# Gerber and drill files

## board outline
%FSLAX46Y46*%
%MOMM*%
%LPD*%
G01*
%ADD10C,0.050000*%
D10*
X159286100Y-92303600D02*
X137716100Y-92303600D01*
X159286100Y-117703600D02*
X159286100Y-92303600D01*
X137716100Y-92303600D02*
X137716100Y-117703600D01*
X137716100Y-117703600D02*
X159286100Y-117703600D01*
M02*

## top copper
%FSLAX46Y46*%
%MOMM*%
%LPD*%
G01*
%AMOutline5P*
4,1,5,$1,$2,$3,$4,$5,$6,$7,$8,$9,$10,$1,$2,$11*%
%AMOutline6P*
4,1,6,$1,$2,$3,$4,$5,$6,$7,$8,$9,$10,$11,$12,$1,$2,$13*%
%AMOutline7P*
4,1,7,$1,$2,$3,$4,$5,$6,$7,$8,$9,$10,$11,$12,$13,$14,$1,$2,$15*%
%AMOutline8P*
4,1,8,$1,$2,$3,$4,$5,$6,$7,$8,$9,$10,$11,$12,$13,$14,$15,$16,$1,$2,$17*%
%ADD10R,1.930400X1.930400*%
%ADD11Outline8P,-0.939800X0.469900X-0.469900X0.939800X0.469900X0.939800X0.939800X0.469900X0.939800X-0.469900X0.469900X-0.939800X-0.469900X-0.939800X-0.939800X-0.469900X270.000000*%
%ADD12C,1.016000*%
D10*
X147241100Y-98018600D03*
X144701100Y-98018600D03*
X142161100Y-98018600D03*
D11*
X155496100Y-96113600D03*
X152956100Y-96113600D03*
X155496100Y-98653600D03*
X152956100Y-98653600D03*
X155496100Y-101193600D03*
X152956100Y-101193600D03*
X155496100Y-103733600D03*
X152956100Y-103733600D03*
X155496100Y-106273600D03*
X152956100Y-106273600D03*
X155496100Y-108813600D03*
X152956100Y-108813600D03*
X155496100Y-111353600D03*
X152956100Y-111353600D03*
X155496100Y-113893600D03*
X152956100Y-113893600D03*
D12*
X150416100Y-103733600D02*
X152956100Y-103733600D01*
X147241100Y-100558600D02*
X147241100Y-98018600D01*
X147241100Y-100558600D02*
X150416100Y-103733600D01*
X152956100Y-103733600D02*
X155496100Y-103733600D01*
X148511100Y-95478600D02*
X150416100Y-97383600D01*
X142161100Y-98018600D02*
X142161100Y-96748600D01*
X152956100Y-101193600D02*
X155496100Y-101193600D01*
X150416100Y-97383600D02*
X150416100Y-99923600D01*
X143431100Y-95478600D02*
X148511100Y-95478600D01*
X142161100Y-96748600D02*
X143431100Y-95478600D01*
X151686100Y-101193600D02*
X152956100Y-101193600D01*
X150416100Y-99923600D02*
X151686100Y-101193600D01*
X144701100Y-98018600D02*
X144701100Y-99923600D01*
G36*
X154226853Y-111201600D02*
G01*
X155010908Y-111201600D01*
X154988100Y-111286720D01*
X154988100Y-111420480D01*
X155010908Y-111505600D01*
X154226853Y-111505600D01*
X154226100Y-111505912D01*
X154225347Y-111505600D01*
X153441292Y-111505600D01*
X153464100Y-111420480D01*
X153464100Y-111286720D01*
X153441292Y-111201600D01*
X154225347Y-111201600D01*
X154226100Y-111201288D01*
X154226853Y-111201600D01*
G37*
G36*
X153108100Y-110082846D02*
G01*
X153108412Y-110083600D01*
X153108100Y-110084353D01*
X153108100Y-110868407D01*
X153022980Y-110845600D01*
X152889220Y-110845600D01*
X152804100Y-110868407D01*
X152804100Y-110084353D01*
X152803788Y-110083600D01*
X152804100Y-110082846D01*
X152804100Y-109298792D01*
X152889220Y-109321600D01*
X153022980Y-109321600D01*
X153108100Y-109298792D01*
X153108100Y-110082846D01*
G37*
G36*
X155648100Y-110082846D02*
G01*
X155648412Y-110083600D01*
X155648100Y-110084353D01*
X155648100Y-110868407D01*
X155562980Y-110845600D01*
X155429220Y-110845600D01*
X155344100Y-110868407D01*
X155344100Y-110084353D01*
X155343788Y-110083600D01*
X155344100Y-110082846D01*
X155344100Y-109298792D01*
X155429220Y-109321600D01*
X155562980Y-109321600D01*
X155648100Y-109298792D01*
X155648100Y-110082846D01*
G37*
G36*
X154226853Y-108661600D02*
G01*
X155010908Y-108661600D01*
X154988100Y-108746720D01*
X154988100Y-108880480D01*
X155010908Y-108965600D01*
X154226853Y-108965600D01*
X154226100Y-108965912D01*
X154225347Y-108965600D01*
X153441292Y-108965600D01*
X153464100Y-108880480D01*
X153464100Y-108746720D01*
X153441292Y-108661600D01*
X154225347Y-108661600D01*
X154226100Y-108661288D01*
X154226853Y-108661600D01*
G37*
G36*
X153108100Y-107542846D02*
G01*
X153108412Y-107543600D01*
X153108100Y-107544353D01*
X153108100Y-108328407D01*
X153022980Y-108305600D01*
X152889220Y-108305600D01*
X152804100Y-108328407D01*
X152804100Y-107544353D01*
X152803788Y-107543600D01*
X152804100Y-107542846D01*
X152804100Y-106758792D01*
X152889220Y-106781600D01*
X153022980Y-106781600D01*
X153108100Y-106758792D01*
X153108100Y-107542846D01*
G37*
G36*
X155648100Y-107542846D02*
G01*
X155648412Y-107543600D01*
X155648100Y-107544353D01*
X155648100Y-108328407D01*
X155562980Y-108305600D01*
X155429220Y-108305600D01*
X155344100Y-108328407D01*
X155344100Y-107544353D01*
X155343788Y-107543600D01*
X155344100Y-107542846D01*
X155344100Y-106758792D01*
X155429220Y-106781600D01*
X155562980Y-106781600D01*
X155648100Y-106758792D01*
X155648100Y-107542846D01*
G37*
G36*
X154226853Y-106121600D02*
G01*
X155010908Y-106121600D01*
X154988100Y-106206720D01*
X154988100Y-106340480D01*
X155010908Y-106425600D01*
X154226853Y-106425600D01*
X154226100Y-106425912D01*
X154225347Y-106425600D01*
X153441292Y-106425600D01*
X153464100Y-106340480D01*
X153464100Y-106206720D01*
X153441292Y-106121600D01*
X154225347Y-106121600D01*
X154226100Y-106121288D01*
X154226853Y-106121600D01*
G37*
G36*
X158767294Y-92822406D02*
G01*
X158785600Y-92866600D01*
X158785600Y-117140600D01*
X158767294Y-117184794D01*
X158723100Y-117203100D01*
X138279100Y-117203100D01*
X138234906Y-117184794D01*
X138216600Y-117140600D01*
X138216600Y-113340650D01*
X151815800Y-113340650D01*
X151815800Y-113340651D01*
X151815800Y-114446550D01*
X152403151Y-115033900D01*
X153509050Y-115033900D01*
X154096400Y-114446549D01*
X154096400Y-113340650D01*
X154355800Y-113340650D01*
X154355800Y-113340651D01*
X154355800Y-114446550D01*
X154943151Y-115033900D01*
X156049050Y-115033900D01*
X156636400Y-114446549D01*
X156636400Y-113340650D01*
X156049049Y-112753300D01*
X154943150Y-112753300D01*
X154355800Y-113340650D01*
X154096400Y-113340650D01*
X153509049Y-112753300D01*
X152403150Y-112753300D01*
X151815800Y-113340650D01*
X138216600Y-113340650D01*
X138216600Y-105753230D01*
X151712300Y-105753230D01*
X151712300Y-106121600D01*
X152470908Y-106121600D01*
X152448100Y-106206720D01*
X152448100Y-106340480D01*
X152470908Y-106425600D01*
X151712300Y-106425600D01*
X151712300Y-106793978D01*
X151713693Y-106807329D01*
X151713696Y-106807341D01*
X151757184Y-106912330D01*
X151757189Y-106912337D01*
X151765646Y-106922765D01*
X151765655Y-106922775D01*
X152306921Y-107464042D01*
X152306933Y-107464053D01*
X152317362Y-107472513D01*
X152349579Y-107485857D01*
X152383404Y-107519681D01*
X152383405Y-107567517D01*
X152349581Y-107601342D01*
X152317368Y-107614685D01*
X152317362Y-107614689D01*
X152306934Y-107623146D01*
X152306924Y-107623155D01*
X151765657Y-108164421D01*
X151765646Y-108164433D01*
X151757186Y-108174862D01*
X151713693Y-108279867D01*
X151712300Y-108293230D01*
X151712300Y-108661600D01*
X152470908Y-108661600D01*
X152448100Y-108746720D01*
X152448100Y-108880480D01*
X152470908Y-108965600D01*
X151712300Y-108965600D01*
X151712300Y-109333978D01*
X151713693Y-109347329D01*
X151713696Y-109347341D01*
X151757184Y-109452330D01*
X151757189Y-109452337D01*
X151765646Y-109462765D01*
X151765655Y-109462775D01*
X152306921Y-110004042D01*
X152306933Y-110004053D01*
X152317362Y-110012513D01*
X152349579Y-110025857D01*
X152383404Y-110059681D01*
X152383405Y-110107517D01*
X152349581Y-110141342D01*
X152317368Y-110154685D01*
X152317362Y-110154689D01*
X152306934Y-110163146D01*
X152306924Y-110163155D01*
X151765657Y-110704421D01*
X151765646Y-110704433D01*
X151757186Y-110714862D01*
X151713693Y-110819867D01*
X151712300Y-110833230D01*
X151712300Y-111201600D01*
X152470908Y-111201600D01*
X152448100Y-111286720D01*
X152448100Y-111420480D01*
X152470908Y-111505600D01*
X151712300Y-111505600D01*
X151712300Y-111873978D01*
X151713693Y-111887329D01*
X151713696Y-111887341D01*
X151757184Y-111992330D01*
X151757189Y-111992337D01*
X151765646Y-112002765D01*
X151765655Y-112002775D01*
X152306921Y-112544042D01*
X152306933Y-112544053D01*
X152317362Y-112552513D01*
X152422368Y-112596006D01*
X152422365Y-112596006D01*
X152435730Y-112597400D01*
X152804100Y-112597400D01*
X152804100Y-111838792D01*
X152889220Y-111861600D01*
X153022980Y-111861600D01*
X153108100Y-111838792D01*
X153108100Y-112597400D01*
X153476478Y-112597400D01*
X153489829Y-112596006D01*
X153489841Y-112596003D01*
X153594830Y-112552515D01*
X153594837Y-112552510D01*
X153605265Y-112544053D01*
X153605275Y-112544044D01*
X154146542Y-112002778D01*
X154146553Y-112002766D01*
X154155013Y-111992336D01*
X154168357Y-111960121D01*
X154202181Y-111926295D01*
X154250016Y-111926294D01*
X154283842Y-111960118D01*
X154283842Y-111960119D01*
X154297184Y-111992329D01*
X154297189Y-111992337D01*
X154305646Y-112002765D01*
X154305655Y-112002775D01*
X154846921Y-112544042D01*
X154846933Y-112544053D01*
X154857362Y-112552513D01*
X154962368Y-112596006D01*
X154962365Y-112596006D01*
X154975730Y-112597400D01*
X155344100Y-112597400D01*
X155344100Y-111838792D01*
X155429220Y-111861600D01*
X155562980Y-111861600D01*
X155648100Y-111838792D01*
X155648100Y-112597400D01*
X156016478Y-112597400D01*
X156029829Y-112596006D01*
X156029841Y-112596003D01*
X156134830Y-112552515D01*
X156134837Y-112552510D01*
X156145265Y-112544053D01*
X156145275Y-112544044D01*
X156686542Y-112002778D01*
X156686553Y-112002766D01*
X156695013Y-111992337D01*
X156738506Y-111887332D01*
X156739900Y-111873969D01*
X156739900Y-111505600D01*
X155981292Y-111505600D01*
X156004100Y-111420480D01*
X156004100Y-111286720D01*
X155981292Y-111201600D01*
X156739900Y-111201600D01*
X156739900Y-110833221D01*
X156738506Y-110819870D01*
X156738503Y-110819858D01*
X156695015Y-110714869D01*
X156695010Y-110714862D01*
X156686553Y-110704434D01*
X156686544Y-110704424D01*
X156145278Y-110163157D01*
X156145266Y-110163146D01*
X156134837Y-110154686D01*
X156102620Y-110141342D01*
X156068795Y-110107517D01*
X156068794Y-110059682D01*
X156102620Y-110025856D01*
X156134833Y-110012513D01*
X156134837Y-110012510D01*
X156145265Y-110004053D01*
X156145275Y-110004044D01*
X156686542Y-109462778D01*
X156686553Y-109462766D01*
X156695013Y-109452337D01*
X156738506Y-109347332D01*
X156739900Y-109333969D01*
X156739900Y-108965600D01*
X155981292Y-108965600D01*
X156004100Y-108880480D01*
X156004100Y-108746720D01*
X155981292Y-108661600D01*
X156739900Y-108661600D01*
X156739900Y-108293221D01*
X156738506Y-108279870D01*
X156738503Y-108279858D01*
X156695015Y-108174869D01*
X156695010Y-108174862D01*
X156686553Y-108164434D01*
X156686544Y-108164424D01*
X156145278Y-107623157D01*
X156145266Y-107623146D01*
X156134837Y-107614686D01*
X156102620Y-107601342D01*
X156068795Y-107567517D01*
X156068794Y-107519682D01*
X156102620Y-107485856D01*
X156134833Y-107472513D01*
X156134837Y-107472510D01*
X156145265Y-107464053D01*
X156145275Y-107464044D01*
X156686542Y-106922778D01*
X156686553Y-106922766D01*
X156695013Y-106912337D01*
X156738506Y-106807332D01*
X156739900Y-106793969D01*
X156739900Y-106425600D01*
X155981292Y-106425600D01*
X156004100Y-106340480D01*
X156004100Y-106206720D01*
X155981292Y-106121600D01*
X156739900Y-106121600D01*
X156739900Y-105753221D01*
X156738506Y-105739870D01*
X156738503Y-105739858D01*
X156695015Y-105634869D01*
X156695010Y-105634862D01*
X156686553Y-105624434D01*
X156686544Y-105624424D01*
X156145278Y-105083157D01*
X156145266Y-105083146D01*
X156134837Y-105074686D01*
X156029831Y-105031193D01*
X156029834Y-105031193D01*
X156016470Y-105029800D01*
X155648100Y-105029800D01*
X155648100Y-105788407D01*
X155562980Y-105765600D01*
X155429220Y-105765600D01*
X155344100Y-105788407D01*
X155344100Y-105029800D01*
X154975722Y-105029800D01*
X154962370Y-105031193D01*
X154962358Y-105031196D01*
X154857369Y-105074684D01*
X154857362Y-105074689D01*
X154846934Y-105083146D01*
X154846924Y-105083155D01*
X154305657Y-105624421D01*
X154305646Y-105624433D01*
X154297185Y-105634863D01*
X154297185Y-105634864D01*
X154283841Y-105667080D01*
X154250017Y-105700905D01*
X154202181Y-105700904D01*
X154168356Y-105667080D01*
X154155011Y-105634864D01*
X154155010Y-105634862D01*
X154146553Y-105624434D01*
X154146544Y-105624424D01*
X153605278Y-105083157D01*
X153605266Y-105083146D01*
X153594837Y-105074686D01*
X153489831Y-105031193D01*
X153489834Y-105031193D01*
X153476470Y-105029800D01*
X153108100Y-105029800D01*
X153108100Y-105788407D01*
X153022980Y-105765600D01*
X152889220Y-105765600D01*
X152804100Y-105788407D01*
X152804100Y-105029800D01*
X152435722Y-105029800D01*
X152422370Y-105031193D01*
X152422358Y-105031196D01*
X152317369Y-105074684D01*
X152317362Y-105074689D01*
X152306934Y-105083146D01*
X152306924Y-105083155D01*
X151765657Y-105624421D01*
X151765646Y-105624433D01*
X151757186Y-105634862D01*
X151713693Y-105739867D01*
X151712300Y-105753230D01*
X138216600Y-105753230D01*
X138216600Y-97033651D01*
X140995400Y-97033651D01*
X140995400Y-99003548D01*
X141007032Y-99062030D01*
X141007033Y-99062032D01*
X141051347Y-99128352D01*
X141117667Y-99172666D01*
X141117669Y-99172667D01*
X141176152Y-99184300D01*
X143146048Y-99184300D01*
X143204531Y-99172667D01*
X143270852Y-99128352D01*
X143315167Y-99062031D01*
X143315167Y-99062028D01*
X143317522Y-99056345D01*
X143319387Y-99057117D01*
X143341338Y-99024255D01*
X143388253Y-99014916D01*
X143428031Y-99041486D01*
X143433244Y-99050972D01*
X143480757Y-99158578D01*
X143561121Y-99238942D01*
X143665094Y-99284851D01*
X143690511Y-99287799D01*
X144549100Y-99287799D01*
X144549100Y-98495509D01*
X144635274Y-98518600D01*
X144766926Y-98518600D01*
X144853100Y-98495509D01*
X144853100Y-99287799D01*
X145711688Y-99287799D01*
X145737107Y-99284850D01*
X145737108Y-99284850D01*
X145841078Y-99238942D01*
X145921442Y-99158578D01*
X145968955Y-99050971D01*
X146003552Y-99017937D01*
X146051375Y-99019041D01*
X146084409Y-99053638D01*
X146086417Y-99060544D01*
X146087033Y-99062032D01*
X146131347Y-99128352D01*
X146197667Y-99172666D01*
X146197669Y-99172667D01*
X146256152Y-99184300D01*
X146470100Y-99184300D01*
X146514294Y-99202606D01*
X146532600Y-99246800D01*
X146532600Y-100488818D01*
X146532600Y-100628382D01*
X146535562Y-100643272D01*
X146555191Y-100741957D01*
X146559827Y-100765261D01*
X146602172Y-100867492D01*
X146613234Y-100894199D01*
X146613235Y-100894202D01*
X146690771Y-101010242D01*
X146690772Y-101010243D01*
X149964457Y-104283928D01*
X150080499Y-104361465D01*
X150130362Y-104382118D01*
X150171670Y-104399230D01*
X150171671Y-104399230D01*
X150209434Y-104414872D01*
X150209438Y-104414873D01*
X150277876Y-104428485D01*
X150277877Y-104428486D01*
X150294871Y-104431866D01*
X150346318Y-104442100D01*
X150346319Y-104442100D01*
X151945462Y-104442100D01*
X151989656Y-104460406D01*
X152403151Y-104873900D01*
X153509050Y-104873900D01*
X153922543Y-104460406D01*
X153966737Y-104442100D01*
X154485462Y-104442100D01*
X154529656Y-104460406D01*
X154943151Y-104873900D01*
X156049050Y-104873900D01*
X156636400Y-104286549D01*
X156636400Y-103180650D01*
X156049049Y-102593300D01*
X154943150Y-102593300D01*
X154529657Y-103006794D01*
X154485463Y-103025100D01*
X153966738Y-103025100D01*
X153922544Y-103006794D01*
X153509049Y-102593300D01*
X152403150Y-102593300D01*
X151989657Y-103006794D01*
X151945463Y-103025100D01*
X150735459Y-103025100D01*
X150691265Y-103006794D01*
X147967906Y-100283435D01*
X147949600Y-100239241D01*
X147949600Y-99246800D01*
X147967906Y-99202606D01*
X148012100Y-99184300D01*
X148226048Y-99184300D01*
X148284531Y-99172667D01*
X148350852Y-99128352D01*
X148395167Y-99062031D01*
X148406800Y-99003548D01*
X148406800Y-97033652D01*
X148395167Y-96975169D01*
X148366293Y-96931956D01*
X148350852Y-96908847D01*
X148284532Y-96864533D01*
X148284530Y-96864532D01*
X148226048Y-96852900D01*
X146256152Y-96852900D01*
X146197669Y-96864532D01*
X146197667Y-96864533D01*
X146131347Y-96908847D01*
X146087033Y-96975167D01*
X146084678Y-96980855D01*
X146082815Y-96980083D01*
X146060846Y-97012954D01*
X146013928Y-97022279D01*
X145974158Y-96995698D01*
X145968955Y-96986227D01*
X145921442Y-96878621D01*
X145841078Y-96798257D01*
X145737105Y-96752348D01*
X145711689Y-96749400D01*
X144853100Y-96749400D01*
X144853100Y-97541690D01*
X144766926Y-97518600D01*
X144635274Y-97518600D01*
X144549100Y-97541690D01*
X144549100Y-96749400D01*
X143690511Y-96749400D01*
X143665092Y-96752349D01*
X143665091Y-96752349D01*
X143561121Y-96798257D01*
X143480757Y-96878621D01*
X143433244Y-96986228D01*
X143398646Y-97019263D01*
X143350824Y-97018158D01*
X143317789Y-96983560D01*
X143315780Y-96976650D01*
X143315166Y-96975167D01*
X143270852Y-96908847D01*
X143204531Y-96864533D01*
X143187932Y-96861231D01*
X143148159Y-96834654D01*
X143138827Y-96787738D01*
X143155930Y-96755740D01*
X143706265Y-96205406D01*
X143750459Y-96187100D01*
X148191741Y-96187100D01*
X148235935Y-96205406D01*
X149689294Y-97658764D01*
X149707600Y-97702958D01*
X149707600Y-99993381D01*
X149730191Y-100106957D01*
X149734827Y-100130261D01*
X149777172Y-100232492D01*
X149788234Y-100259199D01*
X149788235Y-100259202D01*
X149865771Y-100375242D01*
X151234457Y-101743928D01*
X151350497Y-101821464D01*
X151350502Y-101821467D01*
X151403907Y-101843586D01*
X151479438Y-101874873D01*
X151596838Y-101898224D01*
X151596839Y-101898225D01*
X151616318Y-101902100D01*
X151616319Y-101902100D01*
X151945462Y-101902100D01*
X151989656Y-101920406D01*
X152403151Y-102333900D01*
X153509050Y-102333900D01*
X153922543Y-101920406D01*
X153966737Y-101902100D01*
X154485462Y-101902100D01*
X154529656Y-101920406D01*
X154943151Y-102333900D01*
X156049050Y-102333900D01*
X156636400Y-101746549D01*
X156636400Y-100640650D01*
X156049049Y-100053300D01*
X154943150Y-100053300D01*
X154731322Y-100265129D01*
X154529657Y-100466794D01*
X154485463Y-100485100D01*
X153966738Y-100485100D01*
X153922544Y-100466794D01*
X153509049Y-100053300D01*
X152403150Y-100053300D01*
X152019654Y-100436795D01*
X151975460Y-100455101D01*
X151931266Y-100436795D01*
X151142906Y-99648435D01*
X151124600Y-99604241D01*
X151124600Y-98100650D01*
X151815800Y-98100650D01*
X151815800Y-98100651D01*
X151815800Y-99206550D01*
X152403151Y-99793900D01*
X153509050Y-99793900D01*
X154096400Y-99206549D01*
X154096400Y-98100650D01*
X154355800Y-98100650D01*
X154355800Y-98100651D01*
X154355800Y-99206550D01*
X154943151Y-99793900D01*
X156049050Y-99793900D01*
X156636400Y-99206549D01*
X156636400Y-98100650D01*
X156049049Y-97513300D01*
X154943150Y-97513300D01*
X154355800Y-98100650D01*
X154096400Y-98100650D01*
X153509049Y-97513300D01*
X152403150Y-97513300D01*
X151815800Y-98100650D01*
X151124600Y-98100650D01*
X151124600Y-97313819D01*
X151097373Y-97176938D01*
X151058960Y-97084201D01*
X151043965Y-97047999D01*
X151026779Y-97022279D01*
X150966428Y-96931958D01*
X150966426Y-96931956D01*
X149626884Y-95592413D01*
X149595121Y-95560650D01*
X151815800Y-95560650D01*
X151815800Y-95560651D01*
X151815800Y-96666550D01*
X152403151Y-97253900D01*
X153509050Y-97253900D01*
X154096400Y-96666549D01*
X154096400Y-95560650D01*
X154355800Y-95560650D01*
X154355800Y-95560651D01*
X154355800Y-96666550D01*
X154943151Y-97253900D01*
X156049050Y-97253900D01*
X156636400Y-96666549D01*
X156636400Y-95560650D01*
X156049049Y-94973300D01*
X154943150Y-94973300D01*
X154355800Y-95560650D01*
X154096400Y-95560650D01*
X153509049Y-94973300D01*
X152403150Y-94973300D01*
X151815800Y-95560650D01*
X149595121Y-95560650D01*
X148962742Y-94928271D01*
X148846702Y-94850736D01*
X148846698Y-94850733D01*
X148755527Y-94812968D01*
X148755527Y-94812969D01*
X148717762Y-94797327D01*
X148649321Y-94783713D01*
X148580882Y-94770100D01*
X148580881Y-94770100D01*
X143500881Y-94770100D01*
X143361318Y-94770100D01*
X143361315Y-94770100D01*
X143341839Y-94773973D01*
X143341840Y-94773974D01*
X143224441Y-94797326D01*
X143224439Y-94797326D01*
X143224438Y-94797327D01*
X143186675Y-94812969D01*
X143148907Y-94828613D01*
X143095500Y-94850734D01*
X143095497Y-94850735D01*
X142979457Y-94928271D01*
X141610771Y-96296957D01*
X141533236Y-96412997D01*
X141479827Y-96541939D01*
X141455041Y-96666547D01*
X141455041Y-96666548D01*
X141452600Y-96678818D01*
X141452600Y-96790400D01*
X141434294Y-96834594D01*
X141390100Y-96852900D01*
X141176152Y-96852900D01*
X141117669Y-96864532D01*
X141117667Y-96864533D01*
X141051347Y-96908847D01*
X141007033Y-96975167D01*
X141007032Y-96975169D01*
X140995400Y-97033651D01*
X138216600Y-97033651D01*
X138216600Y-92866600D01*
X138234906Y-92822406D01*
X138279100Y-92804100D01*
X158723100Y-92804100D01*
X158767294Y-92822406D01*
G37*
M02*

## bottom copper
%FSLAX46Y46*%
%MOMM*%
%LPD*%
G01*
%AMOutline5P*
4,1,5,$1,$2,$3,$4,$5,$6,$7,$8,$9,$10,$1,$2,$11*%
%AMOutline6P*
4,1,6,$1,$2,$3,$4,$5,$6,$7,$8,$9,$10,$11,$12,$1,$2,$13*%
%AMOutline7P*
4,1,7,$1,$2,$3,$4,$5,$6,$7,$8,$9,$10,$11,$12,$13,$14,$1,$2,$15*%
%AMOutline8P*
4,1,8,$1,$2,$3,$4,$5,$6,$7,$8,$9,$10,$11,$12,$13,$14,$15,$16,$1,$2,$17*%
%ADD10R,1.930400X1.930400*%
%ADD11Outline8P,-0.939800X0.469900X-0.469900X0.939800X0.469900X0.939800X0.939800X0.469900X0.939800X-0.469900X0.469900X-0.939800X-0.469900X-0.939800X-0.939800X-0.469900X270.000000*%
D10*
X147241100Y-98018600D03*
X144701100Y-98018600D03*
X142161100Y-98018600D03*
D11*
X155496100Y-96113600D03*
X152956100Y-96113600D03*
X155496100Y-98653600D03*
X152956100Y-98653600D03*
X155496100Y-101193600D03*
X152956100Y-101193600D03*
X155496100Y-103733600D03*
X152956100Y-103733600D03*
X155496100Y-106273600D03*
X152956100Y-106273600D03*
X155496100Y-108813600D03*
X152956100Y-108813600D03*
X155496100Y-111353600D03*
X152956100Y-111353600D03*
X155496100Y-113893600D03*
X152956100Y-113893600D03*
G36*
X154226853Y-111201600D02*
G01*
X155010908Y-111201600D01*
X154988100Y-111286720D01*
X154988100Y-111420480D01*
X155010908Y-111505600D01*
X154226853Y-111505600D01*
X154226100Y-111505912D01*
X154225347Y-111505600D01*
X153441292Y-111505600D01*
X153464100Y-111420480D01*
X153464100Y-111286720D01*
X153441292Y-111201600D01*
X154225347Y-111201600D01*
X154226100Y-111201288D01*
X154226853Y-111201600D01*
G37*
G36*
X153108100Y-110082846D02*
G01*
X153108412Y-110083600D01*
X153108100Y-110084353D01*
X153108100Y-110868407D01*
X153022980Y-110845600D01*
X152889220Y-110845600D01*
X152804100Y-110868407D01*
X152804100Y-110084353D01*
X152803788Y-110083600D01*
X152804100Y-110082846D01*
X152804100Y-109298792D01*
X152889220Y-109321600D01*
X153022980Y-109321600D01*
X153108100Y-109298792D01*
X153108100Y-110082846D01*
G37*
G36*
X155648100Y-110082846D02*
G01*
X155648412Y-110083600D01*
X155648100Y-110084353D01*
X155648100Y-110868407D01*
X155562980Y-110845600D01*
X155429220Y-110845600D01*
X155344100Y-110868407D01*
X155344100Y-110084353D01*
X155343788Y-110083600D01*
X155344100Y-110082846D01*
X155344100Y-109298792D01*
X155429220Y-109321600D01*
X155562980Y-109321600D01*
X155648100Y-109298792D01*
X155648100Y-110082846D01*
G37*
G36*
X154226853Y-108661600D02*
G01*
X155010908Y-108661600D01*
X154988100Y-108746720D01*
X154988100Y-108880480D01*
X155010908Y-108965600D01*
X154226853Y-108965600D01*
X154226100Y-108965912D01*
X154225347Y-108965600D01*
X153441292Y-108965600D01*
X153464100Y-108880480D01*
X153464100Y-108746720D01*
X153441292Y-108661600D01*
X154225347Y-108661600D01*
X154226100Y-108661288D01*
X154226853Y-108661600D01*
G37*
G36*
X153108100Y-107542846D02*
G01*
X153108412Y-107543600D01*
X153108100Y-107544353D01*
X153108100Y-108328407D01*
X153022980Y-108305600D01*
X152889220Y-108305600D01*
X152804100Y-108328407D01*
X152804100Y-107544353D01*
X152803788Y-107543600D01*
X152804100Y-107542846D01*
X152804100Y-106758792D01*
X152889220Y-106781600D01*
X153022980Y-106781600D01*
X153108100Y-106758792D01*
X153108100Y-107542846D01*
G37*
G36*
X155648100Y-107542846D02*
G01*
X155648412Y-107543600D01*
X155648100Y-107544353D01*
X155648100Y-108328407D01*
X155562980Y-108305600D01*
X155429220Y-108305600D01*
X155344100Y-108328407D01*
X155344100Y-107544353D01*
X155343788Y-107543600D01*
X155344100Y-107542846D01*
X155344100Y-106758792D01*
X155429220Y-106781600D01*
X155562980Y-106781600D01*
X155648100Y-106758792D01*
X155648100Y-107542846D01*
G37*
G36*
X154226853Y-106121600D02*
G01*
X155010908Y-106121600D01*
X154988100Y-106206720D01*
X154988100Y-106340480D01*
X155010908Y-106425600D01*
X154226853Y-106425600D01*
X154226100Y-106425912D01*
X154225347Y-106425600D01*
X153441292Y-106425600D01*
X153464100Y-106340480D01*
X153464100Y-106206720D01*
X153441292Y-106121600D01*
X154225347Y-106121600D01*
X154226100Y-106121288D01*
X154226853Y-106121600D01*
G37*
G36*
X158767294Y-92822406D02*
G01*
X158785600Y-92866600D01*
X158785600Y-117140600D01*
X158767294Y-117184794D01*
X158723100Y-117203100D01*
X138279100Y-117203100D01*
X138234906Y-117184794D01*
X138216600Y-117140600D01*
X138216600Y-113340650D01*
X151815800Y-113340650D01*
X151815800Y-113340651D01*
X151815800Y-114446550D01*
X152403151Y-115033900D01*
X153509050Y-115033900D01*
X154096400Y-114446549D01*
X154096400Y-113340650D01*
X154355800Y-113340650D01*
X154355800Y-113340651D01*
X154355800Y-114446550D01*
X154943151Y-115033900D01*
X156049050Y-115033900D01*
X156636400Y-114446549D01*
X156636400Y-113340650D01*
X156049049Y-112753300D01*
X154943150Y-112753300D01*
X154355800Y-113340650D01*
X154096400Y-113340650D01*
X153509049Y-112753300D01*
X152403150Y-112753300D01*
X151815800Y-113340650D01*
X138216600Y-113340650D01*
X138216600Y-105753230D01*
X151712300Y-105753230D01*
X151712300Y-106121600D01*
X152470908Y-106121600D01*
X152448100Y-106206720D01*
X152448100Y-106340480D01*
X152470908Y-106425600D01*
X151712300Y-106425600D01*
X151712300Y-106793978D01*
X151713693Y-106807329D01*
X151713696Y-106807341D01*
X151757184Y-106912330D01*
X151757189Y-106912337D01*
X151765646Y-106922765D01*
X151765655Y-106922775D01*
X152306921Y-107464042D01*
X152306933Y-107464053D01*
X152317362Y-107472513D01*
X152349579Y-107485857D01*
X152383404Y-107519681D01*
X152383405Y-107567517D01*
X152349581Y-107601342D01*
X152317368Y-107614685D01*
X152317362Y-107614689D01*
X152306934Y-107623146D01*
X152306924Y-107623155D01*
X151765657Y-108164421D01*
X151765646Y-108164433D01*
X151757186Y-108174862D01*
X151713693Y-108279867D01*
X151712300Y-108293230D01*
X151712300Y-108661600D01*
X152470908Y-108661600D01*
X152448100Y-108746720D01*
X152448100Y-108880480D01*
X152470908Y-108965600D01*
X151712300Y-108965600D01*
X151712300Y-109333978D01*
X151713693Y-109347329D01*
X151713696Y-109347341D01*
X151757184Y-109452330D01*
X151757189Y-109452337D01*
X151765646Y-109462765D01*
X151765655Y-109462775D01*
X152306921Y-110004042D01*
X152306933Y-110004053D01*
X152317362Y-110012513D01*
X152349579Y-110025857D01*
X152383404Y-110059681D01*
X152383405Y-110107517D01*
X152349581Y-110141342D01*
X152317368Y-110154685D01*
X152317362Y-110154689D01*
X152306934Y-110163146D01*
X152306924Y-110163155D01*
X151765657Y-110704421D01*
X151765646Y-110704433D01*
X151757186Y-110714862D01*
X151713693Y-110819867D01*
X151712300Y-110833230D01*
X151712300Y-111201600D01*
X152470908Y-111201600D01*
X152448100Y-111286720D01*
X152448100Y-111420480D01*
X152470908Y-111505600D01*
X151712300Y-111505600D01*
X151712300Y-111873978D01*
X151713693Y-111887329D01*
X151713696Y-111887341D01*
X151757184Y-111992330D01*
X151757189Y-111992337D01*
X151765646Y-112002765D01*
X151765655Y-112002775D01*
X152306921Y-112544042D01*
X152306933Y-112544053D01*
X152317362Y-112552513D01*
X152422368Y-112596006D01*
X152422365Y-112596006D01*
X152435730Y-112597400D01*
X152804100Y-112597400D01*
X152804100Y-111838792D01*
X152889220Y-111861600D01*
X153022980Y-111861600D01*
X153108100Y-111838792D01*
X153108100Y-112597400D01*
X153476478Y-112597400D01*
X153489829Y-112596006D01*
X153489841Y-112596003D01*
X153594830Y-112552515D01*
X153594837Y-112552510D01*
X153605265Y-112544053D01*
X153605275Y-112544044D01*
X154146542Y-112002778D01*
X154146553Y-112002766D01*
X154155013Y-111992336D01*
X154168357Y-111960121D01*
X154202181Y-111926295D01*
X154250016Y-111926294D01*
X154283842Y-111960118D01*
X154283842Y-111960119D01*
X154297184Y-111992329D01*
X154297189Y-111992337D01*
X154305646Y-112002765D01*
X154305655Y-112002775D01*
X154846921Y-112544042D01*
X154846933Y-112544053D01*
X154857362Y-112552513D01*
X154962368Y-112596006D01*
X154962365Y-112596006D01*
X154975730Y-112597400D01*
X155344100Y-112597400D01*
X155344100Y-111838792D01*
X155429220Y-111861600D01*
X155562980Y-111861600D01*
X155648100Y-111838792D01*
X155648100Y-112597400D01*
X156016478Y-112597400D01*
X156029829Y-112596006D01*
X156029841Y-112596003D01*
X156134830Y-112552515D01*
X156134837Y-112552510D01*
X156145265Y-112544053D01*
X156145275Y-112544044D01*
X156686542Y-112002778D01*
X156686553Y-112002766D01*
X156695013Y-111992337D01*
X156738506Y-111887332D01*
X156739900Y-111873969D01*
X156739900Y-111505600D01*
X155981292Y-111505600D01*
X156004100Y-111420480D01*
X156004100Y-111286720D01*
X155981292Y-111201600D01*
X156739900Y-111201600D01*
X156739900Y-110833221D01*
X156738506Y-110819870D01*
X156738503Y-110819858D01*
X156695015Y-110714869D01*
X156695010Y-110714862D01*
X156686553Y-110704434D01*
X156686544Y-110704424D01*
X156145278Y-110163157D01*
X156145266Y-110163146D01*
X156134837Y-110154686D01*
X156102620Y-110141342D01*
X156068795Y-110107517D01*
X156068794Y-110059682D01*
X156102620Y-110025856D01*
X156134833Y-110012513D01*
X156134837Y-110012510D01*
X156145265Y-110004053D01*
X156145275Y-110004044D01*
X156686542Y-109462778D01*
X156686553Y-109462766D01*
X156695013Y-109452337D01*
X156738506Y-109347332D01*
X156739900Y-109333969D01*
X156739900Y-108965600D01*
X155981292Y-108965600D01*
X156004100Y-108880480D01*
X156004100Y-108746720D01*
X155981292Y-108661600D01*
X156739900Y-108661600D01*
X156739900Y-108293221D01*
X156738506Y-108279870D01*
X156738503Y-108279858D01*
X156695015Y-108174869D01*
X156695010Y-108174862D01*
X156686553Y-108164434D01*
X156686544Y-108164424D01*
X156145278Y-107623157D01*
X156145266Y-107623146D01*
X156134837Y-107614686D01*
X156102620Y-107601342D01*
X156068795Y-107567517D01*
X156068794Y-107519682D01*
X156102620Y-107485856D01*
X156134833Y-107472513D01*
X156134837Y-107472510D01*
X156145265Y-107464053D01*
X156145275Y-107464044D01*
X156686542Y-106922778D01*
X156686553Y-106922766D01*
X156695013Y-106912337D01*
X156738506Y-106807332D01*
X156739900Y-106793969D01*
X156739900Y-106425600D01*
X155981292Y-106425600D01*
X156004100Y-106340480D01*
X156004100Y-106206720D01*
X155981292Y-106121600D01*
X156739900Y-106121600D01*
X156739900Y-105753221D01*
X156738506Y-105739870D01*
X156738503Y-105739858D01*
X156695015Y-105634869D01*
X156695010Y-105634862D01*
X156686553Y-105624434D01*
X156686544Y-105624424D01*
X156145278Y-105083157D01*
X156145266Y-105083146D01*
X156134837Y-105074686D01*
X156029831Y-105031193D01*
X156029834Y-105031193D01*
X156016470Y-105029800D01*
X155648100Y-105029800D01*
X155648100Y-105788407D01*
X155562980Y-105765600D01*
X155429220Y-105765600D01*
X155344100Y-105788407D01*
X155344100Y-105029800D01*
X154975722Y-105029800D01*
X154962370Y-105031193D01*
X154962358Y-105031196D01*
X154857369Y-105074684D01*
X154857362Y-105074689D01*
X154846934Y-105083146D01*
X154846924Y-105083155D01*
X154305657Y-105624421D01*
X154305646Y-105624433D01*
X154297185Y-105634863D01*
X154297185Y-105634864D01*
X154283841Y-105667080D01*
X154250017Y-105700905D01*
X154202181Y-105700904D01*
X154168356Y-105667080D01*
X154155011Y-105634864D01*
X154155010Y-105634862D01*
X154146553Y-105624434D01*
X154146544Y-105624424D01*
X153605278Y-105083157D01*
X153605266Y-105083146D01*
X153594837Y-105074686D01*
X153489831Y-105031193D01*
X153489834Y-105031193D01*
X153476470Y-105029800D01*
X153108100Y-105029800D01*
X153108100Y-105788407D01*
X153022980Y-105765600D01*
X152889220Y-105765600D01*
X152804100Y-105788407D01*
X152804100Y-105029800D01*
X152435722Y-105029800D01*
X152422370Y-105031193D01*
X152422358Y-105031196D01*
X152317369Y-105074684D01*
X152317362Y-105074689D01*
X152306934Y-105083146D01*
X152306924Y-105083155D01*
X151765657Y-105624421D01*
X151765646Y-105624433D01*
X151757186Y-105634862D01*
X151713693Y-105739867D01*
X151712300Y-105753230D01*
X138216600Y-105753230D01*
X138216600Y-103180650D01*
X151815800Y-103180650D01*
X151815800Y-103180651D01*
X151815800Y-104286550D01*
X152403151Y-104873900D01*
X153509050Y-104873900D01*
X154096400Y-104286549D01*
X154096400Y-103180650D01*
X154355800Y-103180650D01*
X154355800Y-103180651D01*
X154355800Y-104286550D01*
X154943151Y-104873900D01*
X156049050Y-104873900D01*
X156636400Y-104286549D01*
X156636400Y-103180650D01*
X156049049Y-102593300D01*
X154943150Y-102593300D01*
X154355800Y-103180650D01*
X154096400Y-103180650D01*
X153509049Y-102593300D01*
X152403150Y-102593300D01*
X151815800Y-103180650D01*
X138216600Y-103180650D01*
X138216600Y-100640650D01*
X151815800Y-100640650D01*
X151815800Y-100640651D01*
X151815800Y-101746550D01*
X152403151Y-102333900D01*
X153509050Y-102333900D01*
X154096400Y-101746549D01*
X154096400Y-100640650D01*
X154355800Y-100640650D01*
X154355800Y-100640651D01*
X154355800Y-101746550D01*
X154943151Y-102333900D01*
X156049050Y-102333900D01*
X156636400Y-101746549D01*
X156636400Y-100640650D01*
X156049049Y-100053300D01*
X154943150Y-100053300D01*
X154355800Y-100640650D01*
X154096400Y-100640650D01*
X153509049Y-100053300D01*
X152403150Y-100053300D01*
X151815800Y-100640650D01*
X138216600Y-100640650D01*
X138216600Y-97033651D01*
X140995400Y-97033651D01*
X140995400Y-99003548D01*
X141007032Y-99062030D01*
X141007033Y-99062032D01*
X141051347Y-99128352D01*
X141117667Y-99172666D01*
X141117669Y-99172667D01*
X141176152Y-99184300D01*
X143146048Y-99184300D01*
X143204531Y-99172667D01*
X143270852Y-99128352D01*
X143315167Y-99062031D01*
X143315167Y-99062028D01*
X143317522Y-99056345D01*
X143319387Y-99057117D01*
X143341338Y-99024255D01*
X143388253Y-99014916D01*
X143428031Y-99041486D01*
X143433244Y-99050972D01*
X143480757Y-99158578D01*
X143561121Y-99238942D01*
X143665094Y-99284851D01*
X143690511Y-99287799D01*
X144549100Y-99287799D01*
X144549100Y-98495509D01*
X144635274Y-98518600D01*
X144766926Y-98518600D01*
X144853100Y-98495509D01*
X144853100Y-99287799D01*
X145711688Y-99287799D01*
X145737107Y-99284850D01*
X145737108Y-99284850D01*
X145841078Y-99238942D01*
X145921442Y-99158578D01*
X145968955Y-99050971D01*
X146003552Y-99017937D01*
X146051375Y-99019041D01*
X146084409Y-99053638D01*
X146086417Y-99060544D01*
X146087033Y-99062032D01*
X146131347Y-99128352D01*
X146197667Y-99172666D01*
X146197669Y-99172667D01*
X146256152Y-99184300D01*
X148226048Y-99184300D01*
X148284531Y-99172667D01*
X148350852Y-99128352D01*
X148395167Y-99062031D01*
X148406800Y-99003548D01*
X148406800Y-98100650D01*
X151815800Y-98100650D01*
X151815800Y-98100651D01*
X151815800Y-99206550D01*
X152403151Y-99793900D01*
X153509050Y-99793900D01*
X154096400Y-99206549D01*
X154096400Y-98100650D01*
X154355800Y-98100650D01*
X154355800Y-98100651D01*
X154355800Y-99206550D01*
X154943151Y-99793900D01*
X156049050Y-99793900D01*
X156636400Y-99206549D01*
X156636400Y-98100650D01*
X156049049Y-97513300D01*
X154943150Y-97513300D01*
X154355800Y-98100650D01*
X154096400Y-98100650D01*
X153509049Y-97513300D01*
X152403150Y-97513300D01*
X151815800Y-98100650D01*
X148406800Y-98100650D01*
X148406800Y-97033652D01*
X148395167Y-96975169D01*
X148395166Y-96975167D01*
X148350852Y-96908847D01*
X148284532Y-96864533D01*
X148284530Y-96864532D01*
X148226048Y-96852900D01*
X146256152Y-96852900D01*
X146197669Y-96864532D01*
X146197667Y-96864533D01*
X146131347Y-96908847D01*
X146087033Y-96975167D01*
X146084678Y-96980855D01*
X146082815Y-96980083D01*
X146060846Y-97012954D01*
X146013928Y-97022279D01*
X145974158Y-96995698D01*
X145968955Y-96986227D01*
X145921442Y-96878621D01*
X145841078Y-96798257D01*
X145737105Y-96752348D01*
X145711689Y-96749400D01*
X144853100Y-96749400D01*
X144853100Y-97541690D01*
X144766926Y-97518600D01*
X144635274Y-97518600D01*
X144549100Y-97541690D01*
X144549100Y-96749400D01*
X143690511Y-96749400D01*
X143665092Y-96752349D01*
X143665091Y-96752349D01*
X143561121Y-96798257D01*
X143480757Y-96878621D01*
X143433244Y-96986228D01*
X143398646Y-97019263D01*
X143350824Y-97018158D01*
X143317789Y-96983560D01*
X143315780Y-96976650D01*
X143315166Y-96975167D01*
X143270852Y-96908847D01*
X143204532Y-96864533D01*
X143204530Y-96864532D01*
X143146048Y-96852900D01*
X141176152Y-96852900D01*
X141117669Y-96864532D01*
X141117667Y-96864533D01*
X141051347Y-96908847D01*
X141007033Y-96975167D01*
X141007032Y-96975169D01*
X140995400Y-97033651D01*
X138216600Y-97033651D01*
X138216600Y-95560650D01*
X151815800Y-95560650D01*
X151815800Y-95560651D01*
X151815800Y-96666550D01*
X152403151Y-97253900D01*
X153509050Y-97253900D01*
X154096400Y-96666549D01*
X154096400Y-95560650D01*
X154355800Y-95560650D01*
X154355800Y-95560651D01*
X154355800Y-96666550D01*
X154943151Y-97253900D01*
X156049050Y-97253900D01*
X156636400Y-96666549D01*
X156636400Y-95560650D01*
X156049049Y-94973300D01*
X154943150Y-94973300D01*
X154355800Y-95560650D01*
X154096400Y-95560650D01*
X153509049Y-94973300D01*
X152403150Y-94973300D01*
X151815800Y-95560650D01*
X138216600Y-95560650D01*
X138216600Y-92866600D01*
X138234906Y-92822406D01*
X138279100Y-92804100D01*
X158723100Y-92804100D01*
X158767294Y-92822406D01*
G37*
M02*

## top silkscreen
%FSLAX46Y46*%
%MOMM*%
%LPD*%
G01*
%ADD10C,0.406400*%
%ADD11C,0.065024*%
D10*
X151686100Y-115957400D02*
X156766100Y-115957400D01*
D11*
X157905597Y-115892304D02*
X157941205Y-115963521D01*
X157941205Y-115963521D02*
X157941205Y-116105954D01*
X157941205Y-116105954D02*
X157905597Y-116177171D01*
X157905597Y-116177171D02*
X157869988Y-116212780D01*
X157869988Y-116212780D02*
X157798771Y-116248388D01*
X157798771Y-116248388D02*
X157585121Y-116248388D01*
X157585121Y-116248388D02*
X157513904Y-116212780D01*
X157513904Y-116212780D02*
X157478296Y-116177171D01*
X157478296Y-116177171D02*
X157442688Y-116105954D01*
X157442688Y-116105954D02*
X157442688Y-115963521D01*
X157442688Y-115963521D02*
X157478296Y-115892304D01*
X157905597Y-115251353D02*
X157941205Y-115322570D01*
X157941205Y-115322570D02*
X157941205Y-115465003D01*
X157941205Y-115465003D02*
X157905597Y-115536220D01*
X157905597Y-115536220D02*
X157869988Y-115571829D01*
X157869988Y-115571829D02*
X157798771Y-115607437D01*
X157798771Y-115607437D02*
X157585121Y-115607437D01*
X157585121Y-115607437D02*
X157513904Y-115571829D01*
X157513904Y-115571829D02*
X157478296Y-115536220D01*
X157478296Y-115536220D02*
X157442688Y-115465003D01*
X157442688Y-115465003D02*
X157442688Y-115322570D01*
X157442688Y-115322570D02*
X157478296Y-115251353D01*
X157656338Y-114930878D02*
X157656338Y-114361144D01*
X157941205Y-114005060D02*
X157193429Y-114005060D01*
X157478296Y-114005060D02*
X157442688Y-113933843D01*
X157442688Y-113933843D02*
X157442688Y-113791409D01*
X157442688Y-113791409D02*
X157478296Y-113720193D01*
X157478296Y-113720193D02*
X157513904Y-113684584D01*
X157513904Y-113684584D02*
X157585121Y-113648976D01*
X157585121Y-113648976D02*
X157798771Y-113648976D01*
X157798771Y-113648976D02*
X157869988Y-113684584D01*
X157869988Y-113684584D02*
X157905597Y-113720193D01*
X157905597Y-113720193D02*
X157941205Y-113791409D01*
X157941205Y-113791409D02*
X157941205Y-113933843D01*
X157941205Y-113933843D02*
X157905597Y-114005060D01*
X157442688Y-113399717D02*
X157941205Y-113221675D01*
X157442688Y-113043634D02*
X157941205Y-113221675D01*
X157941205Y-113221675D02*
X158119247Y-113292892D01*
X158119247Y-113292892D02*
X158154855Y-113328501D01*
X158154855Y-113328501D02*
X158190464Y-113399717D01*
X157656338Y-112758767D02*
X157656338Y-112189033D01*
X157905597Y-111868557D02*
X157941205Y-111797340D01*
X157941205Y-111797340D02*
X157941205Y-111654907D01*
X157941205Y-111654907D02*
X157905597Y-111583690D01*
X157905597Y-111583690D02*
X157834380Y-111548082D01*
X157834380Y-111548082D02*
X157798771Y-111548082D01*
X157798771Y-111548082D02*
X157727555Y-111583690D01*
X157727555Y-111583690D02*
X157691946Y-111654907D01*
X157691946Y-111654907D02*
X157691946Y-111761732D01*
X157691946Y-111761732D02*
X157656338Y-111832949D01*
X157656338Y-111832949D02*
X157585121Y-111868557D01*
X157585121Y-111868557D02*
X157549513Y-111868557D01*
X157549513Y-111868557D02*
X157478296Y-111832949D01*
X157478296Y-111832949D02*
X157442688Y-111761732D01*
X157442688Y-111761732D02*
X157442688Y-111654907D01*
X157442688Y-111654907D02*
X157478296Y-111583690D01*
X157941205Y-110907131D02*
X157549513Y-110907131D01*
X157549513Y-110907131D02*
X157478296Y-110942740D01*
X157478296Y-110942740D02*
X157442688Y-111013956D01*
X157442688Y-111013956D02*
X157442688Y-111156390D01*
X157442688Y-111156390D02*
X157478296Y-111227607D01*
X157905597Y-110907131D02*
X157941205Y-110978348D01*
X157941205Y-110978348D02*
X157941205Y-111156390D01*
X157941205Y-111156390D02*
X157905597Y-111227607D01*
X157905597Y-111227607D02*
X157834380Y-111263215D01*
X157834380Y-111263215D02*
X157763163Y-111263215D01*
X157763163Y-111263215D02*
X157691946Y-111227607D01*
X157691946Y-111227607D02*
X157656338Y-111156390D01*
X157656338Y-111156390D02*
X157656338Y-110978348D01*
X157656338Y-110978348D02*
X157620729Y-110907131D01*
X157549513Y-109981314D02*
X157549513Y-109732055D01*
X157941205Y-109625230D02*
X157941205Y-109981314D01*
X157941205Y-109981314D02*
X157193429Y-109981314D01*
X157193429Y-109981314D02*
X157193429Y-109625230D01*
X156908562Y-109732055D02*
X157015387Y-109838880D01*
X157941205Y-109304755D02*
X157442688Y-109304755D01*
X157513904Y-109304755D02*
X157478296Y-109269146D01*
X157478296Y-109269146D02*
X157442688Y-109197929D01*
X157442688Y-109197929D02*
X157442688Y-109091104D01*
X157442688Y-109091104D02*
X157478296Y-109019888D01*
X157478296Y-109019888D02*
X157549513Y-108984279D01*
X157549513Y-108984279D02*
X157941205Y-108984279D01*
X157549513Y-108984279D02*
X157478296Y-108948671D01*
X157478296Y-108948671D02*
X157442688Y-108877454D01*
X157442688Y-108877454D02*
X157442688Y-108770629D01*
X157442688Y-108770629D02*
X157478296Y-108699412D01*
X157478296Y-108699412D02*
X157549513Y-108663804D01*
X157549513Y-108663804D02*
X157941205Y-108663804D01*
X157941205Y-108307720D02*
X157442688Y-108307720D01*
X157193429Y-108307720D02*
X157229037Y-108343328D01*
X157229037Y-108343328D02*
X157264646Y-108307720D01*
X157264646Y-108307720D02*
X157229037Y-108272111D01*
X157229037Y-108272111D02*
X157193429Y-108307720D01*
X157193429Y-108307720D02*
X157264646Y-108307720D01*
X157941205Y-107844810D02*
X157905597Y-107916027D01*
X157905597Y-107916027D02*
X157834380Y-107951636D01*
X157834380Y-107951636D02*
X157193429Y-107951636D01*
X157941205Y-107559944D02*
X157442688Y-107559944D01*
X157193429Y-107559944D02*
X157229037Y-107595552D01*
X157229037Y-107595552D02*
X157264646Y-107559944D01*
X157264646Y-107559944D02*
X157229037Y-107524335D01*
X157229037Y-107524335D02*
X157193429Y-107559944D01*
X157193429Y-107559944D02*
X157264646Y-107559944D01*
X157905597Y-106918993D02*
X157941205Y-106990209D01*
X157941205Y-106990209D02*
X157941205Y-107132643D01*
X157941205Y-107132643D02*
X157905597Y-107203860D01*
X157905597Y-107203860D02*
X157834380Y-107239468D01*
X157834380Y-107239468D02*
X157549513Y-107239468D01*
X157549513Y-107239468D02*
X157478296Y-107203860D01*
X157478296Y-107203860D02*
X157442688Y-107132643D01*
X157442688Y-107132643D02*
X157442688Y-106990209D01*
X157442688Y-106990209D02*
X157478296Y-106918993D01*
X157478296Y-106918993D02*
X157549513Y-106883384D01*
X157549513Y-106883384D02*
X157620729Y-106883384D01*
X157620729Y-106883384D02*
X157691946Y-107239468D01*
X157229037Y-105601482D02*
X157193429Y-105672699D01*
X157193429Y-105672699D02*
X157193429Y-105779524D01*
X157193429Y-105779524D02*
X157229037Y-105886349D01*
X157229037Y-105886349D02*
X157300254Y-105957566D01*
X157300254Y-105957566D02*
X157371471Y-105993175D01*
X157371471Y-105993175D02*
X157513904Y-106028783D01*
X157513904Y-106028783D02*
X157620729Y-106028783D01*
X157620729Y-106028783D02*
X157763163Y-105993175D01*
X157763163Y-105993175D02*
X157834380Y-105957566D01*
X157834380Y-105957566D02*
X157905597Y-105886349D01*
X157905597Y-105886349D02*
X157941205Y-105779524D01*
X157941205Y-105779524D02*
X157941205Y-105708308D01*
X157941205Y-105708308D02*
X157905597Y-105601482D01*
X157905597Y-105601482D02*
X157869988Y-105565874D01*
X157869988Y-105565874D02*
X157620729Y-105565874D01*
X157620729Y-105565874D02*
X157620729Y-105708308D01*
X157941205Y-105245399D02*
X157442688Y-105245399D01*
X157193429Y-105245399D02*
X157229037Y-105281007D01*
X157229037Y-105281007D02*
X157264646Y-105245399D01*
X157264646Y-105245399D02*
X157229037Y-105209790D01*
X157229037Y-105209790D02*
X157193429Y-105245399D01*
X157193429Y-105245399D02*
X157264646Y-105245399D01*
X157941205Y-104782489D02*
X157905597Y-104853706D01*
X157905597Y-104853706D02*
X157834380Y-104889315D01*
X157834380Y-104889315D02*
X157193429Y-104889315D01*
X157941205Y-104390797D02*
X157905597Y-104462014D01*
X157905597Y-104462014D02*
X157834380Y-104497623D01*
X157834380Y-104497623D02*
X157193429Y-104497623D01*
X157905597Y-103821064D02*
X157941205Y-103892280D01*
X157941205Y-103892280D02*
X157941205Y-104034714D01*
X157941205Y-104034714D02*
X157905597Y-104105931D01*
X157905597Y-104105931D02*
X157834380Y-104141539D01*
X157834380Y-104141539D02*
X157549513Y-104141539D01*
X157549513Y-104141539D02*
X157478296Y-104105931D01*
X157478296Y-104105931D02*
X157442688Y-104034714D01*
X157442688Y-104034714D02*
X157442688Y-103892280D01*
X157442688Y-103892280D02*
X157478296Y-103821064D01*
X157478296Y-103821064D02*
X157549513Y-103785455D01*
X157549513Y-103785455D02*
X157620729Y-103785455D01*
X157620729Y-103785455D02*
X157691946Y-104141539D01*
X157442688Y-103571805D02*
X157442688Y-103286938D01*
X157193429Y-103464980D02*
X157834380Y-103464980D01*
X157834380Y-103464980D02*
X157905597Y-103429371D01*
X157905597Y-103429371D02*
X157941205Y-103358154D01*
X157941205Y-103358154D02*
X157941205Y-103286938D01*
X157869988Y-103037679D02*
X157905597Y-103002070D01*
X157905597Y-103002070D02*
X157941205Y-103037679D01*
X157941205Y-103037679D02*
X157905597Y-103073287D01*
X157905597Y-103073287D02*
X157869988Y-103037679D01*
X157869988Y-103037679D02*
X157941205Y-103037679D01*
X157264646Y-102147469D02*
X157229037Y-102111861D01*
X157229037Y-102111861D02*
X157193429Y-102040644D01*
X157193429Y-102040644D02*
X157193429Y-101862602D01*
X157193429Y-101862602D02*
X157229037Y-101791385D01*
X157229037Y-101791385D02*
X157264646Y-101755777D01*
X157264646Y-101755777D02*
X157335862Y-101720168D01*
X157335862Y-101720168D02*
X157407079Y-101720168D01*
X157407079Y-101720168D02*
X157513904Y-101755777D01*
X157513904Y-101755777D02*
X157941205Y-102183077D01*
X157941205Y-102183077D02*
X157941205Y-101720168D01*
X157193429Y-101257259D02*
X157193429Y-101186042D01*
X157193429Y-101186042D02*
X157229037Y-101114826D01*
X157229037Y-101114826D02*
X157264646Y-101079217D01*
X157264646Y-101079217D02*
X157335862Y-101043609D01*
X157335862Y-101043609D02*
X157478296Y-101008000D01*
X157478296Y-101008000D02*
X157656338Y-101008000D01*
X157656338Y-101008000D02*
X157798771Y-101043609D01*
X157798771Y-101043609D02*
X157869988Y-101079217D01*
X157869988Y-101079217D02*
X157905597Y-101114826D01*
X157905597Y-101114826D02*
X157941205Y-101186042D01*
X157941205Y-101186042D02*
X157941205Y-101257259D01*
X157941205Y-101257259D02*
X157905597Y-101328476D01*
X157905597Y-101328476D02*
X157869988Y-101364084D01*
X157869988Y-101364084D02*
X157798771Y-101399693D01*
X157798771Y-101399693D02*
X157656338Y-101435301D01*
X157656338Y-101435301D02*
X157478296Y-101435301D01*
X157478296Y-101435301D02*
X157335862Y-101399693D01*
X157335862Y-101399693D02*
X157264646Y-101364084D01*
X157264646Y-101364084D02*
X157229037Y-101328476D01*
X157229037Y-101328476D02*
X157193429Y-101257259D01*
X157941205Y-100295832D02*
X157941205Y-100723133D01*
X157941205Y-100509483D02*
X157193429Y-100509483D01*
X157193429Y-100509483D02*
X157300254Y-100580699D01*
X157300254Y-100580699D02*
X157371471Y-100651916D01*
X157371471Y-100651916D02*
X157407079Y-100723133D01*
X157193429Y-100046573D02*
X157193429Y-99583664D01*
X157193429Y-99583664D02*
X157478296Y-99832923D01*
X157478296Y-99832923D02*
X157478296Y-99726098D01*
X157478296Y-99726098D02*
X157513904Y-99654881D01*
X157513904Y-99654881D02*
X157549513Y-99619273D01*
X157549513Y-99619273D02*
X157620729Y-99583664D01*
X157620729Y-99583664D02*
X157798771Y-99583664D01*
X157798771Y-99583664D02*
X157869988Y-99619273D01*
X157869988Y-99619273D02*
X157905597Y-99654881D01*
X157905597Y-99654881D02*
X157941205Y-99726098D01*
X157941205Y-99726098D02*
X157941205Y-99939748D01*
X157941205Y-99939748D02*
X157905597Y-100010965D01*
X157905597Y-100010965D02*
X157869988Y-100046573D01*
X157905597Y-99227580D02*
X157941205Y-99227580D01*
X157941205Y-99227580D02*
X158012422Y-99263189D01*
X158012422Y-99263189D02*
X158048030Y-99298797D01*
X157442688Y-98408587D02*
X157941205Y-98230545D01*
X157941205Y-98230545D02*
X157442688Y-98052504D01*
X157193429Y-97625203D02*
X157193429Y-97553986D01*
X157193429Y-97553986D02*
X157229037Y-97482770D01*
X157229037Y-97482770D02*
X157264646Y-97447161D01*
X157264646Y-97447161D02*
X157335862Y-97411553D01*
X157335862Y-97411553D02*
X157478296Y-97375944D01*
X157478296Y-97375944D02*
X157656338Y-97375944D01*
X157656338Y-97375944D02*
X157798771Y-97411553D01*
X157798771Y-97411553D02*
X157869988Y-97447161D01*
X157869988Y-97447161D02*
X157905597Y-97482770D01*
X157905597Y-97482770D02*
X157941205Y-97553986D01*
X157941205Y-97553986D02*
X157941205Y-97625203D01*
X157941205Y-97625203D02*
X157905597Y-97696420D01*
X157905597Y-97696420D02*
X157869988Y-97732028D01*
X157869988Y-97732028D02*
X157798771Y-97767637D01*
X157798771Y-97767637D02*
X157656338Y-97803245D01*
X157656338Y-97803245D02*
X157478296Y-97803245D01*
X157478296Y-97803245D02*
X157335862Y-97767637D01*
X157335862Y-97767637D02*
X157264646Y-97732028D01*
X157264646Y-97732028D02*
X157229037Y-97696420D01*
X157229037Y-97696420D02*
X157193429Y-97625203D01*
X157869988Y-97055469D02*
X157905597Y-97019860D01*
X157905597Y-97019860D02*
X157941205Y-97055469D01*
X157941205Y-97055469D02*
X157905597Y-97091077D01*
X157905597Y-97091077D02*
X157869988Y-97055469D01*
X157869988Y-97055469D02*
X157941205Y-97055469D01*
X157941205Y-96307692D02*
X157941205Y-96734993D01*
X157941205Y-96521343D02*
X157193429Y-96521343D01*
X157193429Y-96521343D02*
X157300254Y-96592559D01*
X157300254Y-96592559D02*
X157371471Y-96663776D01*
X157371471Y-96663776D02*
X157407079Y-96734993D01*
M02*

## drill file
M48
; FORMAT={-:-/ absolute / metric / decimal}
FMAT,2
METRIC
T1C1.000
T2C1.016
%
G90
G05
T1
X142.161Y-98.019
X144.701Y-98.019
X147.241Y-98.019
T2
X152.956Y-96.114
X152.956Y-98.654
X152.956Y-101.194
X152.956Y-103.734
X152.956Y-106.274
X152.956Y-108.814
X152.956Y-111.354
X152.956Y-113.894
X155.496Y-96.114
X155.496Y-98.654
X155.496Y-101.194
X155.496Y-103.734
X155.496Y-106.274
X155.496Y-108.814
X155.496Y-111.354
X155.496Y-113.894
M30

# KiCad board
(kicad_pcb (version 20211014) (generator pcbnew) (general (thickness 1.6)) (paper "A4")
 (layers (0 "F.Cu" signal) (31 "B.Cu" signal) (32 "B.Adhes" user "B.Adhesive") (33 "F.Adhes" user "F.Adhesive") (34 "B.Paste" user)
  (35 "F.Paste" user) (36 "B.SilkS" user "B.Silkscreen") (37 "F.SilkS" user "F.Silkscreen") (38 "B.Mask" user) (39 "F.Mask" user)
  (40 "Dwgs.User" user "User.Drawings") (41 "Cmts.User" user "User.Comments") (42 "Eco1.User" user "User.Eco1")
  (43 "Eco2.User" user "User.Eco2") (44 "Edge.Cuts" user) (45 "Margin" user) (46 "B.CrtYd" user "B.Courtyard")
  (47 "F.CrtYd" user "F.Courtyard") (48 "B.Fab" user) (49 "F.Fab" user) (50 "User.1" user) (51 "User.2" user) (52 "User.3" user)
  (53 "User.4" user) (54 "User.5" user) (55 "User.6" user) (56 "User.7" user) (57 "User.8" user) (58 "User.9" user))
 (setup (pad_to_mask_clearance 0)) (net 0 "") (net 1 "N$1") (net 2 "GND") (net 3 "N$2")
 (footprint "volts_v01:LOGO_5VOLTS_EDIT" (layer "F.Cu") (at 139.6211 106.2736)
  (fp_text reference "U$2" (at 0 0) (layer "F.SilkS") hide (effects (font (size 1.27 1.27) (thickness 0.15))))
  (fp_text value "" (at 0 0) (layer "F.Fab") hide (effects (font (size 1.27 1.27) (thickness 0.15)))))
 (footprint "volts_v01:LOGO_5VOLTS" (layer "F.Cu") (at 138.8273 117.2274)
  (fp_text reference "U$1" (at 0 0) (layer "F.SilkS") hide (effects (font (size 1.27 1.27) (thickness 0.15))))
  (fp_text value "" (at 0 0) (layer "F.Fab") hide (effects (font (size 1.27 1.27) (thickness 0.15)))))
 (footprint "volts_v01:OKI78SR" (layer "B.Cu") (at 144.7011 98.0186)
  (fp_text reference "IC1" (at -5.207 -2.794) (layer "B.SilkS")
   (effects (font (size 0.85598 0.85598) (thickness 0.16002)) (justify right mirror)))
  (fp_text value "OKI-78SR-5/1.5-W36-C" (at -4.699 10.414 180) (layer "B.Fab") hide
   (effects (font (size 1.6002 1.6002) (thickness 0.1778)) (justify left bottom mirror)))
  (pad "1" thru_hole rect (at 2.54 0 270) (size 1.9304 1.9304) (drill 1) (layers *.Cu *.Mask) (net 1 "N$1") (solder_mask_margin 0.0762))
  (pad "2" thru_hole rect (at 0 0 270) (size 1.9304 1.9304) (drill 1) (layers *.Cu *.Mask) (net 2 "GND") (solder_mask_margin 0.0762))
  (pad "3" thru_hole rect (at -2.54 0 270) (size 1.9304 1.9304) (drill 1) (layers *.Cu *.Mask) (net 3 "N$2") (solder_mask_margin 0.0762)))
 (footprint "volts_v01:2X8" (layer "B.Cu") (at 155.4961 96.1136 -90)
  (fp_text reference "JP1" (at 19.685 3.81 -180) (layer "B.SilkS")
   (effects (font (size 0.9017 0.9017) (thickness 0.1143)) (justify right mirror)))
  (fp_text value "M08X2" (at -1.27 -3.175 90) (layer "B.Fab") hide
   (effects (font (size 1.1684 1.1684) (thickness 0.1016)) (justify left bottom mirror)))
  (pad "1" thru_hole roundrect (at 0 0 270) (size 1.8796 1.8796) (drill 1.016) (layers *.Cu *.Mask) (roundrect_rratio 0.25)
   (chamfer_ratio 0.25) (chamfer top_left top_right bottom_left bottom_right) (solder_mask_margin 0.0762))
  (pad "2" thru_hole roundrect (at 0 2.54 270) (size 1.8796 1.8796) (drill 1.016) (layers *.Cu *.Mask) (roundrect_rratio 0.25)
   (chamfer_ratio 0.25) (chamfer top_left top_right bottom_left bottom_right) (solder_mask_margin 0.0762))
  (pad "3" thru_hole roundrect (at 2.54 0 270) (size 1.8796 1.8796) (drill 1.016) (layers *.Cu *.Mask) (roundrect_rratio 0.25)
   (chamfer_ratio 0.25) (chamfer top_left top_right bottom_left bottom_right) (solder_mask_margin 0.0762))
  (pad "4" thru_hole roundrect (at 2.54 2.54 270) (size 1.8796 1.8796) (drill 1.016) (layers *.Cu *.Mask) (roundrect_rratio 0.25)
   (chamfer_ratio 0.25) (chamfer top_left top_right bottom_left bottom_right) (solder_mask_margin 0.0762))
  (pad "5" thru_hole roundrect (at 5.08 0 270) (size 1.8796 1.8796) (drill 1.016) (layers *.Cu *.Mask) (roundrect_rratio 0.25)
   (chamfer_ratio 0.25) (chamfer top_left top_right bottom_left bottom_right) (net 3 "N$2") (solder_mask_margin 0.0762))
  (pad "6" thru_hole roundrect (at 5.08 2.54 270) (size 1.8796 1.8796) (drill 1.016) (layers *.Cu *.Mask) (roundrect_rratio 0.25)
   (chamfer_ratio 0.25) (chamfer top_left top_right bottom_left bottom_right) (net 3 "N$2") (solder_mask_margin 0.0762))
  (pad "7" thru_hole roundrect (at 7.62 0 270) (size 1.8796 1.8796) (drill 1.016) (layers *.Cu *.Mask) (roundrect_rratio 0.25)
   (chamfer_ratio 0.25) (chamfer top_left top_right bottom_left bottom_right) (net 1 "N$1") (solder_mask_margin 0.0762))
  (pad "8" thru_hole roundrect (at 7.62 2.54 270) (size 1.8796 1.8796) (drill 1.016) (layers *.Cu *.Mask) (roundrect_rratio 0.25)
   (chamfer_ratio 0.25) (chamfer top_left top_right bottom_left bottom_right) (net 1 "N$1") (solder_mask_margin 0.0762))
  (pad "9" thru_hole roundrect (at 10.16 0 270) (size 1.8796 1.8796) (drill 1.016) (layers *.Cu *.Mask) (roundrect_rratio 0.25)
   (chamfer_ratio 0.25) (chamfer top_left top_right bottom_left bottom_right) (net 2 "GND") (solder_mask_margin 0.0762))
  (pad "10" thru_hole roundrect (at 10.16 2.54 270) (size 1.8796 1.8796) (drill 1.016) (layers *.Cu *.Mask) (roundrect_rratio 0.25)
   (chamfer_ratio 0.25) (chamfer top_left top_right bottom_left bottom_right) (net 2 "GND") (solder_mask_margin 0.0762))
  (pad "11" thru_hole roundrect (at 12.7 0 270) (size 1.8796 1.8796) (drill 1.016) (layers *.Cu *.Mask) (roundrect_rratio 0.25)
   (chamfer_ratio 0.25) (chamfer top_left top_right bottom_left bottom_right) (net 2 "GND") (solder_mask_margin 0.0762))
  (pad "12" thru_hole roundrect (at 12.7 2.54 270) (size 1.8796 1.8796) (drill 1.016) (layers *.Cu *.Mask) (roundrect_rratio 0.25)
   (chamfer_ratio 0.25) (chamfer top_left top_right bottom_left bottom_right) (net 2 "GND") (solder_mask_margin 0.0762))
  (pad "13" thru_hole roundrect (at 15.24 0 270) (size 1.8796 1.8796) (drill 1.016) (layers *.Cu *.Mask) (roundrect_rratio 0.25)
   (chamfer_ratio 0.25) (chamfer top_left top_right bottom_left bottom_right) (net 2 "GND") (solder_mask_margin 0.0762))
  (pad "14" thru_hole roundrect (at 15.24 2.54 270) (size 1.8796 1.8796) (drill 1.016) (layers *.Cu *.Mask) (roundrect_rratio 0.25)
   (chamfer_ratio 0.25) (chamfer top_left top_right bottom_left bottom_right) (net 2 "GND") (solder_mask_margin 0.0762))
  (pad "15" thru_hole roundrect (at 17.78 0 270) (size 1.8796 1.8796) (drill 1.016) (layers *.Cu *.Mask) (roundrect_rratio 0.25)
   (chamfer_ratio 0.25) (chamfer top_left top_right bottom_left bottom_right) (solder_mask_margin 0.0762))
  (pad "16" thru_hole roundrect (at 17.78 2.54 270) (size 1.8796 1.8796) (drill 1.016) (layers *.Cu *.Mask) (roundrect_rratio 0.25)
   (chamfer_ratio 0.25) (chamfer top_left top_right bottom_left bottom_right) (solder_mask_margin 0.0762)))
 (gr_line (start 151.6861 115.9574) (end 156.7661 115.9574) (layer "F.SilkS") (width 0.4064))
 (gr_line (start 159.2861 92.3036) (end 137.7161 92.3036) (layer "Edge.Cuts") (width 0.05))
 (gr_line (start 159.2861 117.7036) (end 159.2861 92.3036) (layer "Edge.Cuts") (width 0.05))
 (gr_line (start 137.7161 92.3036) (end 137.7161 117.7036) (layer "Edge.Cuts") (width 0.05))
 (gr_line (start 137.7161 117.7036) (end 159.2861 117.7036) (layer "Edge.Cuts") (width 0.05))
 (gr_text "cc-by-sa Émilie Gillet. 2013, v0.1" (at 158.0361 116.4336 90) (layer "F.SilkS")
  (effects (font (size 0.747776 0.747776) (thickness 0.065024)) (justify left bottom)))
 (segment (start 150.4161 103.7336) (end 152.9561 103.7336) (width 1.016) (layer "F.Cu") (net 1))
 (segment (start 147.2411 100.5586) (end 147.2411 98.0186) (width 1.016) (layer "F.Cu") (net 1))
 (segment (start 147.2411 100.5586) (end 150.4161 103.7336) (width 1.016) (layer "F.Cu") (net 1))
 (segment (start 152.9561 103.7336) (end 155.4961 103.7336) (width 1.016) (layer "F.Cu") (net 1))
 (segment (start 148.5111 95.4786) (end 150.4161 97.3836) (width 1.016) (layer "F.Cu") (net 3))
 (segment (start 142.1611 98.0186) (end 142.1611 96.7486) (width 1.016) (layer "F.Cu") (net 3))
 (segment (start 152.9561 101.1936) (end 155.4961 101.1936) (width 1.016) (layer "F.Cu") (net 3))
 (segment (start 150.4161 97.3836) (end 150.4161 99.9236) (width 1.016) (layer "F.Cu") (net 3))
 (segment (start 143.4311 95.4786) (end 148.5111 95.4786) (width 1.016) (layer "F.Cu") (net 3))
 (segment (start 142.1611 96.7486) (end 143.4311 95.4786) (width 1.016) (layer "F.Cu") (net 3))
 (segment (start 151.6861 101.1936) (end 152.9561 101.1936) (width 1.016) (layer "F.Cu") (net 3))
 (segment (start 150.4161 99.9236) (end 151.6861 101.1936) (width 1.016) (layer "F.Cu") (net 3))
 (segment (start 144.7011 98.0186) (end 144.7011 99.9236) (width 1.016) (layer "F.Cu") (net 2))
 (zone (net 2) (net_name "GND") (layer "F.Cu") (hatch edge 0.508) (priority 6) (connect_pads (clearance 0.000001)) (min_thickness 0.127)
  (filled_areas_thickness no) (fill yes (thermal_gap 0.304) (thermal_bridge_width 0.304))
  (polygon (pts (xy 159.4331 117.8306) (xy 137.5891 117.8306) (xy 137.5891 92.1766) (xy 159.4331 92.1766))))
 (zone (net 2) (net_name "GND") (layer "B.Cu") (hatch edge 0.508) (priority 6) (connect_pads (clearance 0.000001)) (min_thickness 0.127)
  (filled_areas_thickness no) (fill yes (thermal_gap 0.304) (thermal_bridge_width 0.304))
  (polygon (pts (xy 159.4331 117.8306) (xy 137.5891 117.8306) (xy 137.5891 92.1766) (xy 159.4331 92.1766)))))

